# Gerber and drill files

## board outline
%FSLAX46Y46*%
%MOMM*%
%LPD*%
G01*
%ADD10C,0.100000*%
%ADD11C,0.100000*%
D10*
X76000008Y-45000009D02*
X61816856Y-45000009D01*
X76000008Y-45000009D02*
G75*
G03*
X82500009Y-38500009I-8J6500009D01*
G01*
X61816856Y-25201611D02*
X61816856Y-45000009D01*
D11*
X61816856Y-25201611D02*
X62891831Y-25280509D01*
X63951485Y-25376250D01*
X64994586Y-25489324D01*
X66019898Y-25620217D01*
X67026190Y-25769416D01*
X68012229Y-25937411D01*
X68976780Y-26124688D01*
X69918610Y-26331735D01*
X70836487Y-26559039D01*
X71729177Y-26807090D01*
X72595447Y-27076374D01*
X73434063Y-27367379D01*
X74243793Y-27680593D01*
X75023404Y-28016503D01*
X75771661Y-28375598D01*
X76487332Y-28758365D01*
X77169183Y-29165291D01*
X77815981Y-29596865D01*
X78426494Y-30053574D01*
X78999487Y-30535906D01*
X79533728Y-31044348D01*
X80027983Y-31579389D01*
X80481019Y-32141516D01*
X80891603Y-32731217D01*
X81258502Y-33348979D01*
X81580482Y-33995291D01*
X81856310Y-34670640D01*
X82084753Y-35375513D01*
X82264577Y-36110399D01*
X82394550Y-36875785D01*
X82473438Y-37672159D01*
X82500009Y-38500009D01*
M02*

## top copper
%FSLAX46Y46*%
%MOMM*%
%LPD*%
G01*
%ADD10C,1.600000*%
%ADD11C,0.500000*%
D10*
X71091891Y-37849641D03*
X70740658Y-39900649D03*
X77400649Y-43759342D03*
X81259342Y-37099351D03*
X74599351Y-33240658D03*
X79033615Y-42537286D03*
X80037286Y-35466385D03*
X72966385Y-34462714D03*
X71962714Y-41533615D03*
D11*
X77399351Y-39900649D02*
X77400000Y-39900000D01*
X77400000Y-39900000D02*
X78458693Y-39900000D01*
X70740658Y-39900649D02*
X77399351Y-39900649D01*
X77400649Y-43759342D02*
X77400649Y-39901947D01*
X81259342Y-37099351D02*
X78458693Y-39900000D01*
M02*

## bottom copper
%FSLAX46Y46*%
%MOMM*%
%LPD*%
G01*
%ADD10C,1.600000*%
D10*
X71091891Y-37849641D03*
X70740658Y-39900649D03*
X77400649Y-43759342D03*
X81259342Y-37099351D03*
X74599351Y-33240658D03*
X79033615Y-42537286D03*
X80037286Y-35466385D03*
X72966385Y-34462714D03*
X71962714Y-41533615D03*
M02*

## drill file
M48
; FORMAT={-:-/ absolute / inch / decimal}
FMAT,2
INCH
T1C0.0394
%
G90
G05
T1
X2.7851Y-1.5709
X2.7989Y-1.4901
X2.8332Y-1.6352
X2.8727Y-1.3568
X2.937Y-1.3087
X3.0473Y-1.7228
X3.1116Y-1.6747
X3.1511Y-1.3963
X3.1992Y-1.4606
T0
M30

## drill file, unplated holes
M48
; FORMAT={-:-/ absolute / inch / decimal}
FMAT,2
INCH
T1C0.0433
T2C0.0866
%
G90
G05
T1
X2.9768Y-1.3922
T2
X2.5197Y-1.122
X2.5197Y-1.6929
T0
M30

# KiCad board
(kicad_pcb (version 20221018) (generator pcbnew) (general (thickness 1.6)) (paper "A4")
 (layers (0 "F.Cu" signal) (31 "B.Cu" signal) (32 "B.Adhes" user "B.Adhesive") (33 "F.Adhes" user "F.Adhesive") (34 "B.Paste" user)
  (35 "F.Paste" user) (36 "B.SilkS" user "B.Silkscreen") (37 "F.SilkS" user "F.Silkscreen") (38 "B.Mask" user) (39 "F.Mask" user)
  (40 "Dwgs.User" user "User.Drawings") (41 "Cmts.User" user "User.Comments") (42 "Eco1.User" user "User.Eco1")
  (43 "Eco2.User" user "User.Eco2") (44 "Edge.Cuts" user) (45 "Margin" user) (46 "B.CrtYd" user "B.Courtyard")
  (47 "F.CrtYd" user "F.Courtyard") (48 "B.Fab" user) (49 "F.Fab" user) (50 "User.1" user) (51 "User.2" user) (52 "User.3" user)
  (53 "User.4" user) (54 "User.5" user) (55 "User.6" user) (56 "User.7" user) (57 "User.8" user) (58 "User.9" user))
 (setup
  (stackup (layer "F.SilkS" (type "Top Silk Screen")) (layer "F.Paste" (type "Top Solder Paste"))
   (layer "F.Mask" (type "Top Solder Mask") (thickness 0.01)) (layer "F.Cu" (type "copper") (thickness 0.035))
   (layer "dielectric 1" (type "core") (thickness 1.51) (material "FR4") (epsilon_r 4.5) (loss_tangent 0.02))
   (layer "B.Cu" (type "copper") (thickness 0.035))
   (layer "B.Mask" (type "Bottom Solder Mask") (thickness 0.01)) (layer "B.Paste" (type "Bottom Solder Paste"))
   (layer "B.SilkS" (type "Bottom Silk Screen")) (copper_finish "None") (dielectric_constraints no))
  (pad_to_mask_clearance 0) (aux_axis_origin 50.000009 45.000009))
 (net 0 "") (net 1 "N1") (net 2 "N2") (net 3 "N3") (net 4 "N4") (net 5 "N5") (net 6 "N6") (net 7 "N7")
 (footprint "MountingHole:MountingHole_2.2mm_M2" (layer "F.Cu") (at 64 43)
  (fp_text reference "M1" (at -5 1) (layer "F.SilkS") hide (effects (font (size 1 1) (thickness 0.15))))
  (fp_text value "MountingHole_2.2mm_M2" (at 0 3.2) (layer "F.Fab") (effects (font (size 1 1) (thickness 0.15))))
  (pad "" np_thru_hole circle (at 0 0) (size 2.2 2.2) (drill 2.2) (layers "*.Cu" "*.Mask")))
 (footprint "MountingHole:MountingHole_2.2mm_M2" (layer "F.Cu") (at 64 28.5)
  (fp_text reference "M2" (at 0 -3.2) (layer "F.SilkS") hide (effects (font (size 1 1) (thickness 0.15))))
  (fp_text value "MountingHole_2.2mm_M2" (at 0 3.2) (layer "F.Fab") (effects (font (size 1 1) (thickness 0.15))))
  (pad "" np_thru_hole circle (at 0 0) (size 2.2 2.2) (drill 2.2) (layers "*.Cu" "*.Mask")))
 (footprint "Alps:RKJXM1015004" (layer "F.Cu") (at 76 38.5 25.5)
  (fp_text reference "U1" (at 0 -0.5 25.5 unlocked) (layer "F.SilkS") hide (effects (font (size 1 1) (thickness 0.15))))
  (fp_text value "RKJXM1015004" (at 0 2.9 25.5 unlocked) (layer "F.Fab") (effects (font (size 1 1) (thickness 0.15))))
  (pad "" np_thru_hole circle (at 1 -3 25.5) (size 1.1 1.1) (drill 1.1) (layers "F&B.Cu" "*.Mask"))
  (pad "1" thru_hole circle (at -4.15 -2.7 25.5) (size 1.6 1.6) (drill 1) (layers "*.Cu" "*.Mask") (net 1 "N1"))
  (pad "2" thru_hole circle (at -5.35 -1 25.5) (size 1.6 1.6) (drill 1) (layers "*.Cu" "*.Mask") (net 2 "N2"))
  (pad "2" thru_hole circle (at -1 5.35 25.5) (size 1.6 1.6) (drill 1) (layers "*.Cu" "*.Mask") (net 2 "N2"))
  (pad "2" thru_hole circle (at 5.35 1 25.5) (size 1.6 1.6) (drill 1) (layers "*.Cu" "*.Mask") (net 2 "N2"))
  (pad "3" thru_hole circle (at 1 -5.35 25.5) (size 1.6 1.6) (drill 1) (layers "*.Cu" "*.Mask") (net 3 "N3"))
  (pad "4" thru_hole circle (at 1 4.95 25.5) (size 1.6 1.6) (drill 1) (layers "*.Cu" "*.Mask") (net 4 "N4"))
  (pad "5" thru_hole circle (at 4.95 -1 25.5) (size 1.6 1.6) (drill 1) (layers "*.Cu" "*.Mask") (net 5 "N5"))
  (pad "6" thru_hole circle (at -1 -4.95 25.5) (size 1.6 1.6) (drill 1) (layers "*.Cu" "*.Mask") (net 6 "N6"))
  (pad "7" thru_hole circle (at -4.95 1 25.5) (size 1.6 1.6) (drill 1) (layers "*.Cu" "*.Mask") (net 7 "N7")))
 (gr_line (start 76.000008 45.000009) (end 61.816856 45.000009) (stroke (width 0.1) (type solid)) (layer "Edge.Cuts"))
 (gr_arc (start 82.500009 38.500009) (mid 80.5962 43.096201) (end 76.000008 45.000009) (stroke (width 0.1) (type solid)) (layer "Edge.Cuts"))
 (gr_line (start 61.816856 25.201611) (end 61.816856 45.000009) (stroke (width 0.1) (type solid)) (layer "Edge.Cuts"))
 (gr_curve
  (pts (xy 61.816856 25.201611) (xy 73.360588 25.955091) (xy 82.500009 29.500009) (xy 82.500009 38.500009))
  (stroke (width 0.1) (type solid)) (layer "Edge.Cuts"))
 (segment (start 77.399351 39.900649) (end 77.4 39.9) (width 0.5) (layer "F.Cu") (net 2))
 (segment (start 77.4 39.9) (end 78.458693 39.9) (width 0.5) (layer "F.Cu") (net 2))
 (segment (start 70.740658 39.900649) (end 77.399351 39.900649) (width 0.5) (layer "F.Cu") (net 2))
 (segment (start 77.400649 43.759342) (end 77.400649 39.901947) (width 0.5) (layer "F.Cu") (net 2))
 (segment (start 81.259342 37.099351) (end 78.458693 39.9) (width 0.5) (layer "F.Cu") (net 2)))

